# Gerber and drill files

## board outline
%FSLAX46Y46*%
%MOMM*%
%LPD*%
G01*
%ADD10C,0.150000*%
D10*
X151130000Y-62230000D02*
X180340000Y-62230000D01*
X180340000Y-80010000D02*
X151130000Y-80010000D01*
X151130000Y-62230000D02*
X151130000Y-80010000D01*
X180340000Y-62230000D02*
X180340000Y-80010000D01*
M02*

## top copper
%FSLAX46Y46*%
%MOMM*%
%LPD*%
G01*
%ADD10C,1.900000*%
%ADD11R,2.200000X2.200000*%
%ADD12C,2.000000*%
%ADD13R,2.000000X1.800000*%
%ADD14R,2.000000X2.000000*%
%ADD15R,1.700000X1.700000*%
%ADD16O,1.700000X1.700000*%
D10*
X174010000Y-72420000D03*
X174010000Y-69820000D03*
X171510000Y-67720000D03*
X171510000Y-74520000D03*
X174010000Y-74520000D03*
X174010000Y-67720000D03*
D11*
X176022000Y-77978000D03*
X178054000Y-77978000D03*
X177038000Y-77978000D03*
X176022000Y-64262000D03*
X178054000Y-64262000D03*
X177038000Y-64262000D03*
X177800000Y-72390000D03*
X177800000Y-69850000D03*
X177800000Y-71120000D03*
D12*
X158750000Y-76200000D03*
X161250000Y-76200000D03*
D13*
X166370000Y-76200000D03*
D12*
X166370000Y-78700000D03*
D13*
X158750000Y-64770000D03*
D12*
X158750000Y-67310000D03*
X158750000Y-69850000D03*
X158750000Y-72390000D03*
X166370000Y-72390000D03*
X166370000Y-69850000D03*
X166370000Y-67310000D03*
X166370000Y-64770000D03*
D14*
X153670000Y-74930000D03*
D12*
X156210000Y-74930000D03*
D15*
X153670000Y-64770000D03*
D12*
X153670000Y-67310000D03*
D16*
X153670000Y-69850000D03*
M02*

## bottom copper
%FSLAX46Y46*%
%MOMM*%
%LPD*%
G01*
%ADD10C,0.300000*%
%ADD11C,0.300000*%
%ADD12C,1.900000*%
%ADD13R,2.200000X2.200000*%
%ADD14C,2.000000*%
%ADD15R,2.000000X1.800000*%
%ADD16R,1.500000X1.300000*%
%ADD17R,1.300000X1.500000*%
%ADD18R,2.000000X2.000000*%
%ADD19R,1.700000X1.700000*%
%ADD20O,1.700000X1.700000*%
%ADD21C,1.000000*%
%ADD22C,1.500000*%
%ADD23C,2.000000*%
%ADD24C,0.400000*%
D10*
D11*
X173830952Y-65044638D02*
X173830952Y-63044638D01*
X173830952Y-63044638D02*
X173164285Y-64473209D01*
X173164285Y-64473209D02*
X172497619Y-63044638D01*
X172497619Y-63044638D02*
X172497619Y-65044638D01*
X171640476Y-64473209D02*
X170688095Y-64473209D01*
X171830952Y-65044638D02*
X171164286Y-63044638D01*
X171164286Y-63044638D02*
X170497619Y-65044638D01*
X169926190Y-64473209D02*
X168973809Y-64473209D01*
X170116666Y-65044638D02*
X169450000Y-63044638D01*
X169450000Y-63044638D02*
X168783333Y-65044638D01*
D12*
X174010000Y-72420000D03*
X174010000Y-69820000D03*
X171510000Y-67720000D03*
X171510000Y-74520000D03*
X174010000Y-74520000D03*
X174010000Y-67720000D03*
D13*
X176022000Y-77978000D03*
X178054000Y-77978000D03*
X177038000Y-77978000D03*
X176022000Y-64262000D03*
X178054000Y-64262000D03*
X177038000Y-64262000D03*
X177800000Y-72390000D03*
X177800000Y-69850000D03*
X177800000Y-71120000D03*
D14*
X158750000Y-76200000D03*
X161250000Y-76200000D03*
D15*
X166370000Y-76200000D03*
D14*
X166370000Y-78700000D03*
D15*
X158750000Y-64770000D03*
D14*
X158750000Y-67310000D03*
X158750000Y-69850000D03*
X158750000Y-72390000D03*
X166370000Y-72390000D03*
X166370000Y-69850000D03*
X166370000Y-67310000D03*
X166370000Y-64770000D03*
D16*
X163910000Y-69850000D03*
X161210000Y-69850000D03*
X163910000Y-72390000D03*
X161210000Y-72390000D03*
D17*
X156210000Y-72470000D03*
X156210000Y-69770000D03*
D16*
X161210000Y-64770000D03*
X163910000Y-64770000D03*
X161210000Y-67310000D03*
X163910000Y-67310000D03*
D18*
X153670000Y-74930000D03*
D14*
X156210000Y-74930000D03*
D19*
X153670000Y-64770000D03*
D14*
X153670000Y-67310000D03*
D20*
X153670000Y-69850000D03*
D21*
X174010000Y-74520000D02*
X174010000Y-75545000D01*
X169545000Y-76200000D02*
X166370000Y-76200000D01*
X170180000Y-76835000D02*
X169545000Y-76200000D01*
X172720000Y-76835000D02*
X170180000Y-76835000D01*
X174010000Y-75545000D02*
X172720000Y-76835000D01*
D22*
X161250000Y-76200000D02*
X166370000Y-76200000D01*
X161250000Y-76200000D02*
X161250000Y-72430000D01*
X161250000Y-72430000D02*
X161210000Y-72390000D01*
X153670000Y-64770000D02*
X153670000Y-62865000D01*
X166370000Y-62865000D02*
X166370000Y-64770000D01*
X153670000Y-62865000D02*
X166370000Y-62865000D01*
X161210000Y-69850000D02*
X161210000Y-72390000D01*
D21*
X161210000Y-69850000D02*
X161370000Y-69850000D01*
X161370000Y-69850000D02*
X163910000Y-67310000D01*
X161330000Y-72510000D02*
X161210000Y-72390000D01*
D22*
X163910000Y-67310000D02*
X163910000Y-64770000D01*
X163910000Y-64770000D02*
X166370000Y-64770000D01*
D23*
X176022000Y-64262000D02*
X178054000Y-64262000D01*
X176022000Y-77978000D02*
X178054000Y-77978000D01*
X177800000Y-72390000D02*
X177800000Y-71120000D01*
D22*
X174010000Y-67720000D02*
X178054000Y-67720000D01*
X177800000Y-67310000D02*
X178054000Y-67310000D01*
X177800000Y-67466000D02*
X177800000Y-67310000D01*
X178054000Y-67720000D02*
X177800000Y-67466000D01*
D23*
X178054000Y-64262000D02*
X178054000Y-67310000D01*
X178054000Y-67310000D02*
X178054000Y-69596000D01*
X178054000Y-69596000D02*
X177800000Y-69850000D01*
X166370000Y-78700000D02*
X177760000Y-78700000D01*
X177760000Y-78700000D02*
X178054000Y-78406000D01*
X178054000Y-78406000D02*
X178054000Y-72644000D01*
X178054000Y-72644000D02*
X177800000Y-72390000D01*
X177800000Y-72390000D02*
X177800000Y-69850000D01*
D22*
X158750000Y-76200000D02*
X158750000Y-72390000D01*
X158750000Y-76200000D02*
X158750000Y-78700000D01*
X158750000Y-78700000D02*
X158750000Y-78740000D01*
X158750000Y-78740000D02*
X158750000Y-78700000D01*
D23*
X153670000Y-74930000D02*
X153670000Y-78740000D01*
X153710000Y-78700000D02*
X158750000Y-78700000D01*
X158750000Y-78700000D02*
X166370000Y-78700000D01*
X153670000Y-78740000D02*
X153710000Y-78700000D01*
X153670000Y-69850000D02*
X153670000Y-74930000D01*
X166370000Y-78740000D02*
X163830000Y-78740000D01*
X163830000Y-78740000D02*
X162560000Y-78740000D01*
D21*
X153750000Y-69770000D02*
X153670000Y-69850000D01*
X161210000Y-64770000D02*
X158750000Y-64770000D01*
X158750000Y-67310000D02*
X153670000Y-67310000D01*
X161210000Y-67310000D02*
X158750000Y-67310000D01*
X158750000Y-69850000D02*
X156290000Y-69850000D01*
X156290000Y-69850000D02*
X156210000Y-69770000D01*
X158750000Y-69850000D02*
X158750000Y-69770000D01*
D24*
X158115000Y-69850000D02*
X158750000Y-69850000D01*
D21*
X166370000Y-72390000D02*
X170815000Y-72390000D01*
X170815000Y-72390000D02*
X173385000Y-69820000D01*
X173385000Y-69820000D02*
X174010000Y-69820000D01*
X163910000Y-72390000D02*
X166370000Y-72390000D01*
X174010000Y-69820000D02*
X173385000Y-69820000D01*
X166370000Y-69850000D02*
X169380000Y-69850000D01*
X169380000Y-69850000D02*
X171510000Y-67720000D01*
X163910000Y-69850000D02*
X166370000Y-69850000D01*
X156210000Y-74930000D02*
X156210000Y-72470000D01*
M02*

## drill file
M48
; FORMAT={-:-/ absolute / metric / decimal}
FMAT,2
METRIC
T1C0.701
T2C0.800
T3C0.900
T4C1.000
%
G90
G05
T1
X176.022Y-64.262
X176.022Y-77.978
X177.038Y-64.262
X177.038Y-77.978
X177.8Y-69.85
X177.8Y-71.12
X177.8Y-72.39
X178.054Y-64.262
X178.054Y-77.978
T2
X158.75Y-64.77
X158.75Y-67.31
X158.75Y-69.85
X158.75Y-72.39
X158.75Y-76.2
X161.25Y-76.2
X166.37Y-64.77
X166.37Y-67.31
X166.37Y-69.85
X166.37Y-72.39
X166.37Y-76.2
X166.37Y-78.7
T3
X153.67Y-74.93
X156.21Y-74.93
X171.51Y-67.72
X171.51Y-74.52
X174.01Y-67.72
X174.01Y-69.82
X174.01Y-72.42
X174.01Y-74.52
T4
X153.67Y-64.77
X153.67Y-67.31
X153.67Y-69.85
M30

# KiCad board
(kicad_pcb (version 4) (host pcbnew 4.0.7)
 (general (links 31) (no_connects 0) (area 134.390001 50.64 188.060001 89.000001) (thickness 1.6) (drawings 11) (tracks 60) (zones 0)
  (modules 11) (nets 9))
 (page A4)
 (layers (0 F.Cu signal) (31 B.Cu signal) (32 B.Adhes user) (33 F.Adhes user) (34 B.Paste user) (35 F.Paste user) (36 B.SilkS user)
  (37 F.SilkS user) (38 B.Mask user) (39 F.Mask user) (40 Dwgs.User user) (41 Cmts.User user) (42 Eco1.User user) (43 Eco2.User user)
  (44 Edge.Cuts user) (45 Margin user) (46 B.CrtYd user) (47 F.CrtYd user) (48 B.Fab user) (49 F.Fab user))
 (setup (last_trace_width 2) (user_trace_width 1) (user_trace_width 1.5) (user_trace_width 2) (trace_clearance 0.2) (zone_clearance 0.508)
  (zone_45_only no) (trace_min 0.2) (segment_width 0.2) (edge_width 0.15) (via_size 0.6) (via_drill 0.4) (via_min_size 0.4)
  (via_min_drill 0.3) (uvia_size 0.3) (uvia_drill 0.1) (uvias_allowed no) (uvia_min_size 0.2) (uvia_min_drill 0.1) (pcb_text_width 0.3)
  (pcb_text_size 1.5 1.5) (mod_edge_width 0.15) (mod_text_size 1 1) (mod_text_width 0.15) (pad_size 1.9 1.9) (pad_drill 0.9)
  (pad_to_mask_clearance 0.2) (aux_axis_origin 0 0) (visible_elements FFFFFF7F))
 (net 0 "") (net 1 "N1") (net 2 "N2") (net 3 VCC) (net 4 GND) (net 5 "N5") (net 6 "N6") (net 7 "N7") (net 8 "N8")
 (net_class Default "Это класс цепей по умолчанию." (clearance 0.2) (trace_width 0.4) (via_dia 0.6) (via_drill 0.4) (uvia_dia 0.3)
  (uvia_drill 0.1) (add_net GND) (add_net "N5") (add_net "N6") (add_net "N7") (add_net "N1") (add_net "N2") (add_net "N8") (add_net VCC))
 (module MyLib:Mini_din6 (layer F.Cu) (at 175.26 71.12 90)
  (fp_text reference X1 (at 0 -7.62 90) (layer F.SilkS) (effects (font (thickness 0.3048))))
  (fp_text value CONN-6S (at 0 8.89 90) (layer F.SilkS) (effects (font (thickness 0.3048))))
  (pad 2 thru_hole circle (at -1.3 -1.25 90) (size 1.9 1.9) (drill 0.9) (layers *.Cu *.Mask F.SilkS))
  (pad 1 thru_hole circle (at 1.3 -1.25 90) (size 1.9 1.9) (drill 0.9) (layers *.Cu *.Mask F.SilkS) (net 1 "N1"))
  (pad 5 thru_hole circle (at 3.4 -3.75 90) (size 1.9 1.9) (drill 0.9) (layers *.Cu *.Mask F.SilkS) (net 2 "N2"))
  (pad 6 thru_hole circle (at -3.4 -3.75 90) (size 1.9 1.9) (drill 0.9) (layers *.Cu *.Mask F.SilkS))
  (pad 4 thru_hole circle (at -3.4 -1.25 90) (size 1.9 1.9) (drill 0.9) (layers *.Cu *.Mask F.SilkS) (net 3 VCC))
  (pad 3 thru_hole circle (at 3.4 -1.25 90) (size 1.9 1.9) (drill 0.9) (layers *.Cu *.Mask F.SilkS) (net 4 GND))
  (pad S thru_hole rect (at -6.858 0.762 90) (size 2.2 2.2) (drill 0.70104) (layers *.Cu *.SilkS *.Mask) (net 4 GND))
  (pad S thru_hole rect (at -6.858 2.794 90) (size 2.2 2.2) (drill 0.70104) (layers *.Cu *.SilkS *.Mask) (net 4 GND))
  (pad S thru_hole rect (at -6.858 1.778 90) (size 2.2 2.2) (drill 0.70104) (layers *.Cu *.SilkS *.Mask) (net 4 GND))
  (pad S thru_hole rect (at 6.858 0.762 90) (size 2.2 2.2) (drill 0.70104) (layers *.Cu *.SilkS *.Mask) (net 4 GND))
  (pad S thru_hole rect (at 6.858 2.794 90) (size 2.2 2.2) (drill 0.70104) (layers *.Cu *.SilkS *.Mask) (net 4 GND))
  (pad S thru_hole rect (at 6.858 1.778 90) (size 2.2 2.2) (drill 0.70104) (layers *.Cu *.SilkS *.Mask) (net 4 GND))
  (pad S thru_hole rect (at -1.27 2.54 90) (size 2.2 2.2) (drill 0.70104) (layers *.Cu *.SilkS *.Mask) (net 4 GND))
  (pad S thru_hole rect (at 1.27 2.54 90) (size 2.2 2.2) (drill 0.70104) (layers *.Cu *.SilkS *.Mask) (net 4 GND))
  (pad S thru_hole rect (at 0 2.54 90) (size 2.2 2.2) (drill 0.70104) (layers *.Cu *.SilkS *.Mask) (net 4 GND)))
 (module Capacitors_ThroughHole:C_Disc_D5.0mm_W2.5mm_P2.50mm (layer F.Cu) (at 158.75 76.2)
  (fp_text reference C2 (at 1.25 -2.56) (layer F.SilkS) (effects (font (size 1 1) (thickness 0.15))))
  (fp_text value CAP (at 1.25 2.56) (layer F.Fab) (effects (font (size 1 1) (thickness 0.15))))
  (pad 1 thru_hole circle (at 0 0) (size 2 2) (drill 0.8) (layers *.Cu *.Mask) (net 4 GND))
  (pad 2 thru_hole circle (at 2.5 0) (size 2 2) (drill 0.8) (layers *.Cu *.Mask) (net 3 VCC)))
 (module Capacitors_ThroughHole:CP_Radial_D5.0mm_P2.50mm (layer F.Cu) (at 166.37 76.2 270)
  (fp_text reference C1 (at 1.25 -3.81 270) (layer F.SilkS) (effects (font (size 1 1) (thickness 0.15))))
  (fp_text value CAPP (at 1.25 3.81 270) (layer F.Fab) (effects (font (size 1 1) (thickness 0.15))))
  (pad 1 thru_hole rect (at 0 0 270) (size 1.8 2) (drill 0.8) (layers *.Cu *.Mask) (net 3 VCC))
  (pad 2 thru_hole circle (at 2.5 0 270) (size 2 2) (drill 0.8) (layers *.Cu *.Mask) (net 4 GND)))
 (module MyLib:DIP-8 (layer F.Cu) (at 158.75 64.77 270)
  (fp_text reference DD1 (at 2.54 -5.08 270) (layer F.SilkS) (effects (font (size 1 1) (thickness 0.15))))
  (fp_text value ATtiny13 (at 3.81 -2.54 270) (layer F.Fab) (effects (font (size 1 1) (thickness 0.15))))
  (pad 1 thru_hole rect (at 0 0 270) (size 1.8 2) (drill 0.8) (layers *.Cu *.Mask F.SilkS) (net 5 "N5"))
  (pad 2 thru_hole circle (at 2.54 0 270) (size 2 2) (drill 0.8) (layers *.Cu *.Mask F.SilkS) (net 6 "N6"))
  (pad 3 thru_hole circle (at 5.08 0 270) (size 2 2) (drill 0.8) (layers *.Cu *.Mask F.SilkS) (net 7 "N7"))
  (pad 4 thru_hole circle (at 7.62 0 270) (size 2 2) (drill 0.8) (layers *.Cu *.Mask F.SilkS) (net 4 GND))
  (pad 5 thru_hole circle (at 7.62 -7.62 270) (size 2 2) (drill 0.8) (layers *.Cu *.Mask F.SilkS) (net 1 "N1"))
  (pad 6 thru_hole circle (at 5.08 -7.62 270) (size 2 2) (drill 0.8) (layers *.Cu *.Mask F.SilkS) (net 2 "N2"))
  (pad 7 thru_hole circle (at 2.54 -7.62 270) (size 2 2) (drill 0.8) (layers *.Cu *.Mask F.SilkS))
  (pad 8 thru_hole circle (at 0 -7.62 270) (size 2 2) (drill 0.8) (layers *.Cu *.Mask F.SilkS) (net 3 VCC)))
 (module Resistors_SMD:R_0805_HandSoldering (layer B.Cu) (at 162.56 69.85 180)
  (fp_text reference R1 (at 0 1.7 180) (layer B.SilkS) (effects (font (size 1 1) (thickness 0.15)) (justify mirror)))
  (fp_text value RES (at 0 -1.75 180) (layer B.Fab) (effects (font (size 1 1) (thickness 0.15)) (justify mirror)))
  (pad 1 smd rect (at -1.35 0 180) (size 1.5 1.3) (layers B.Cu B.Paste B.Mask) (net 2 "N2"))
  (pad 2 smd rect (at 1.35 0 180) (size 1.5 1.3) (layers B.Cu B.Paste B.Mask) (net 3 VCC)))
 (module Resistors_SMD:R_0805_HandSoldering (layer B.Cu) (at 162.56 72.39 180)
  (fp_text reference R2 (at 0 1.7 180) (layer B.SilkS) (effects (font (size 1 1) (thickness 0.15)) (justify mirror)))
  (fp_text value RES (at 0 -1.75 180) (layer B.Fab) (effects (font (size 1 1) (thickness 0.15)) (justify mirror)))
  (pad 1 smd rect (at -1.35 0 180) (size 1.5 1.3) (layers B.Cu B.Paste B.Mask) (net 1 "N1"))
  (pad 2 smd rect (at 1.35 0 180) (size 1.5 1.3) (layers B.Cu B.Paste B.Mask) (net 3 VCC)))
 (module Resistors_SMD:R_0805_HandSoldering (layer B.Cu) (at 156.21 71.12 90)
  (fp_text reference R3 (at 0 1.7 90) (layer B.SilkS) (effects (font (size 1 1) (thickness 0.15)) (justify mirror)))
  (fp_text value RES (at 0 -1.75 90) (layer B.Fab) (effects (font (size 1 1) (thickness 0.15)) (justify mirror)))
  (pad 1 smd rect (at -1.35 0 90) (size 1.5 1.3) (layers B.Cu B.Paste B.Mask) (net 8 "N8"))
  (pad 2 smd rect (at 1.35 0 90) (size 1.5 1.3) (layers B.Cu B.Paste B.Mask) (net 7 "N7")))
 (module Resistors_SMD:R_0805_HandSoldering (layer B.Cu) (at 162.56 64.77)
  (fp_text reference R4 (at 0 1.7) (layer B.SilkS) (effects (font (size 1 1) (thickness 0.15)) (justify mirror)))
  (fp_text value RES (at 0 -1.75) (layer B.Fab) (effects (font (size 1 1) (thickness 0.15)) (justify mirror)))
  (pad 1 smd rect (at -1.35 0) (size 1.5 1.3) (layers B.Cu B.Paste B.Mask) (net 5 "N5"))
  (pad 2 smd rect (at 1.35 0) (size 1.5 1.3) (layers B.Cu B.Paste B.Mask) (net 3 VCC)))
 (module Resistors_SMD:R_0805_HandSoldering (layer B.Cu) (at 162.56 67.31)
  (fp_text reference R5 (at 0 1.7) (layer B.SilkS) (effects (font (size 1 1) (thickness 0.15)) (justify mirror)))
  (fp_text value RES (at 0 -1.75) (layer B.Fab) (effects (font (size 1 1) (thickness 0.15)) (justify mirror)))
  (pad 1 smd rect (at -1.35 0) (size 1.5 1.3) (layers B.Cu B.Paste B.Mask) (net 6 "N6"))
  (pad 2 smd rect (at 1.35 0) (size 1.5 1.3) (layers B.Cu B.Paste B.Mask) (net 3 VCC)))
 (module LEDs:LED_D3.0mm (layer F.Cu) (at 153.67 74.93)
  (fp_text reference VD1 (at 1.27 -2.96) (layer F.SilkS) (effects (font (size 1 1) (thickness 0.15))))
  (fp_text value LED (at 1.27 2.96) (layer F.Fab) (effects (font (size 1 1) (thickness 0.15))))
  (pad 1 thru_hole rect (at 0 0) (size 2 2) (drill 0.9) (layers *.Cu *.Mask) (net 4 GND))
  (pad 2 thru_hole circle (at 2.54 0) (size 2 2) (drill 0.9) (layers *.Cu *.Mask) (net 8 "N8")))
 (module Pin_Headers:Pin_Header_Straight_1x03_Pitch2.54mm (layer F.Cu) (at 153.67 64.77)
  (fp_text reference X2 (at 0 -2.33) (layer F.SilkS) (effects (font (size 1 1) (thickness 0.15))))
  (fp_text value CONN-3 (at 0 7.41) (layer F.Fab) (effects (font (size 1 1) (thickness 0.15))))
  (pad 1 thru_hole rect (at 0 0) (size 1.7 1.7) (drill 1) (layers *.Cu *.Mask) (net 3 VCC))
  (pad 2 thru_hole circle (at 0 2.54) (size 2 2) (drill 1) (layers *.Cu *.Mask) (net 6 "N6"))
  (pad 3 thru_hole oval (at 0 5.08) (size 1.7 1.7) (drill 1) (layers *.Cu *.Mask) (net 4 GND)))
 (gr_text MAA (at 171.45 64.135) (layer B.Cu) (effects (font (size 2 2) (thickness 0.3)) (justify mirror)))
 (gr_line (start 151.13 62.23) (end 180.34 62.23) (angle 90) (layer Edge.Cuts) (width 0.15))
 (gr_line (start 180.34 80.01) (end 151.13 80.01) (angle 90) (layer Edge.Cuts) (width 0.15))
 (gr_line (start 151.13 62.23) (end 151.13 80.01) (angle 90) (layer Edge.Cuts) (width 0.15))
 (gr_line (start 180.34 62.23) (end 180.34 80.01) (angle 90) (layer Edge.Cuts) (width 0.15))
 (segment (start 174.01 74.52) (end 174.01 75.545) (width 1) (layer B.Cu) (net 3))
 (segment (start 169.545 76.2) (end 166.37 76.2) (width 1) (layer B.Cu) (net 3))
 (segment (start 170.18 76.835) (end 169.545 76.2) (width 1) (layer B.Cu) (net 3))
 (segment (start 172.72 76.835) (end 170.18 76.835) (width 1) (layer B.Cu) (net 3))
 (segment (start 174.01 75.545) (end 172.72 76.835) (width 1) (layer B.Cu) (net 3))
 (segment (start 161.25 76.2) (end 166.37 76.2) (width 1.5) (layer B.Cu) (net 3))
 (segment (start 161.25 76.2) (end 161.25 72.43) (width 1.5) (layer B.Cu) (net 3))
 (segment (start 161.25 72.43) (end 161.21 72.39) (width 1.5) (layer B.Cu) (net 3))
 (segment (start 153.67 64.77) (end 153.67 62.865) (width 1.5) (layer B.Cu) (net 3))
 (segment (start 166.37 62.865) (end 166.37 64.77) (width 1.5) (layer B.Cu) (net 3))
 (segment (start 153.67 62.865) (end 166.37 62.865) (width 1.5) (layer B.Cu) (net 3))
 (segment (start 161.21 69.85) (end 161.21 72.39) (width 1.5) (layer B.Cu) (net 3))
 (segment (start 161.21 69.85) (end 161.37 69.85) (width 1) (layer B.Cu) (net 3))
 (segment (start 161.37 69.85) (end 163.91 67.31) (width 1) (layer B.Cu) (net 3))
 (segment (start 161.33 72.51) (end 161.21 72.39) (width 1) (layer B.Cu) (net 3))
 (segment (start 163.91 67.31) (end 163.91 64.77) (width 1.5) (layer B.Cu) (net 3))
 (segment (start 163.91 64.77) (end 166.37 64.77) (width 1.5) (layer B.Cu) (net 3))
 (segment (start 176.022 64.262) (end 178.054 64.262) (width 2) (layer B.Cu) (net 4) (status C00000))
 (segment (start 176.022 77.978) (end 178.054 77.978) (width 2) (layer B.Cu) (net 4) (status C00000))
 (segment (start 177.8 72.39) (end 177.8 71.12) (width 2) (layer B.Cu) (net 4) (status C00000))
 (segment (start 174.01 67.72) (end 178.054 67.72) (width 1.5) (layer B.Cu) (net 4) (status 400000))
 (segment (start 177.8 67.31) (end 178.054 67.31) (width 1.5) (layer B.Cu) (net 4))
 (segment (start 177.8 67.466) (end 177.8 67.31) (width 1.5) (layer B.Cu) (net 4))
 (segment (start 178.054 67.72) (end 177.8 67.466) (width 1.5) (layer B.Cu) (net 4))
 (segment (start 178.054 64.262) (end 178.054 67.31) (width 2) (layer B.Cu) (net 4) (status 400000))
 (segment (start 178.054 67.31) (end 178.054 69.596) (width 2) (layer B.Cu) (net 4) (status 800000))
 (segment (start 178.054 69.596) (end 177.8 69.85) (width 2) (layer B.Cu) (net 4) (status C00000))
 (segment (start 166.37 78.7) (end 177.76 78.7) (width 2) (layer B.Cu) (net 4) (status C00000))
 (segment (start 177.76 78.7) (end 178.054 78.406) (width 2) (layer B.Cu) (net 4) (status C00000))
 (segment (start 178.054 78.406) (end 178.054 72.644) (width 2) (layer B.Cu) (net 4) (status C00000))
 (segment (start 178.054 72.644) (end 177.8 72.39) (width 2) (layer B.Cu) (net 4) (status C00000))
 (segment (start 177.8 72.39) (end 177.8 69.85) (width 2) (layer B.Cu) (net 4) (status C00000))
 (segment (start 158.75 76.2) (end 158.75 72.39) (width 1.5) (layer B.Cu) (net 4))
 (segment (start 158.75 76.2) (end 158.75 78.7) (width 1.5) (layer B.Cu) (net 4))
 (segment (start 158.75 78.7) (end 158.75 78.74) (width 1.5) (layer B.Cu) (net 4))
 (segment (start 158.75 78.74) (end 158.75 78.7) (width 1.5) (layer B.Cu) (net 4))
 (segment (start 153.67 74.93) (end 153.67 78.74) (width 2) (layer B.Cu) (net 4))
 (segment (start 153.71 78.7) (end 158.75 78.7) (width 2) (layer B.Cu) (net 4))
 (segment (start 158.75 78.7) (end 166.37 78.7) (width 2) (layer B.Cu) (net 4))
 (segment (start 153.67 78.74) (end 153.71 78.7) (width 2) (layer B.Cu) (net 4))
 (segment (start 153.67 69.85) (end 153.67 74.93) (width 2) (layer B.Cu) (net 4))
 (segment (start 166.37 78.74) (end 163.83 78.74) (width 2) (layer B.Cu) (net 4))
 (segment (start 163.83 78.74) (end 162.56 78.74) (width 2) (layer B.Cu) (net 4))
 (segment (start 153.75 69.77) (end 153.67 69.85) (width 1) (layer B.Cu) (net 4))
 (segment (start 161.21 64.77) (end 158.75 64.77) (width 1) (layer B.Cu) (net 5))
 (segment (start 158.75 67.31) (end 153.67 67.31) (width 1) (layer B.Cu) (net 6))
 (segment (start 161.21 67.31) (end 158.75 67.31) (width 1) (layer B.Cu) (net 6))
 (segment (start 158.75 69.85) (end 156.29 69.85) (width 1) (layer B.Cu) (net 7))
 (segment (start 156.29 69.85) (end 156.21 69.77) (width 1) (layer B.Cu) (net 7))
 (segment (start 158.75 69.85) (end 158.75 69.77) (width 1) (layer B.Cu) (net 7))
 (segment (start 158.115 69.85) (end 158.75 69.85) (width 0.4) (layer B.Cu) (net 7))
 (segment (start 166.37 72.39) (end 170.815 72.39) (width 1) (layer B.Cu) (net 1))
 (segment (start 170.815 72.39) (end 173.385 69.82) (width 1) (layer B.Cu) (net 1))
 (segment (start 173.385 69.82) (end 174.01 69.82) (width 1) (layer B.Cu) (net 1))
 (segment (start 163.91 72.39) (end 166.37 72.39) (width 1) (layer B.Cu) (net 1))
 (segment (start 174.01 69.82) (end 173.385 69.82) (width 1) (layer B.Cu) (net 1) (status 30))
 (segment (start 166.37 69.85) (end 169.38 69.85) (width 1) (layer B.Cu) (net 2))
 (segment (start 169.38 69.85) (end 171.51 67.72) (width 1) (layer B.Cu) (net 2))
 (segment (start 163.91 69.85) (end 166.37 69.85) (width 1) (layer B.Cu) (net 2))
 (segment (start 156.21 74.93) (end 156.21 72.47) (width 1) (layer B.Cu) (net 8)))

